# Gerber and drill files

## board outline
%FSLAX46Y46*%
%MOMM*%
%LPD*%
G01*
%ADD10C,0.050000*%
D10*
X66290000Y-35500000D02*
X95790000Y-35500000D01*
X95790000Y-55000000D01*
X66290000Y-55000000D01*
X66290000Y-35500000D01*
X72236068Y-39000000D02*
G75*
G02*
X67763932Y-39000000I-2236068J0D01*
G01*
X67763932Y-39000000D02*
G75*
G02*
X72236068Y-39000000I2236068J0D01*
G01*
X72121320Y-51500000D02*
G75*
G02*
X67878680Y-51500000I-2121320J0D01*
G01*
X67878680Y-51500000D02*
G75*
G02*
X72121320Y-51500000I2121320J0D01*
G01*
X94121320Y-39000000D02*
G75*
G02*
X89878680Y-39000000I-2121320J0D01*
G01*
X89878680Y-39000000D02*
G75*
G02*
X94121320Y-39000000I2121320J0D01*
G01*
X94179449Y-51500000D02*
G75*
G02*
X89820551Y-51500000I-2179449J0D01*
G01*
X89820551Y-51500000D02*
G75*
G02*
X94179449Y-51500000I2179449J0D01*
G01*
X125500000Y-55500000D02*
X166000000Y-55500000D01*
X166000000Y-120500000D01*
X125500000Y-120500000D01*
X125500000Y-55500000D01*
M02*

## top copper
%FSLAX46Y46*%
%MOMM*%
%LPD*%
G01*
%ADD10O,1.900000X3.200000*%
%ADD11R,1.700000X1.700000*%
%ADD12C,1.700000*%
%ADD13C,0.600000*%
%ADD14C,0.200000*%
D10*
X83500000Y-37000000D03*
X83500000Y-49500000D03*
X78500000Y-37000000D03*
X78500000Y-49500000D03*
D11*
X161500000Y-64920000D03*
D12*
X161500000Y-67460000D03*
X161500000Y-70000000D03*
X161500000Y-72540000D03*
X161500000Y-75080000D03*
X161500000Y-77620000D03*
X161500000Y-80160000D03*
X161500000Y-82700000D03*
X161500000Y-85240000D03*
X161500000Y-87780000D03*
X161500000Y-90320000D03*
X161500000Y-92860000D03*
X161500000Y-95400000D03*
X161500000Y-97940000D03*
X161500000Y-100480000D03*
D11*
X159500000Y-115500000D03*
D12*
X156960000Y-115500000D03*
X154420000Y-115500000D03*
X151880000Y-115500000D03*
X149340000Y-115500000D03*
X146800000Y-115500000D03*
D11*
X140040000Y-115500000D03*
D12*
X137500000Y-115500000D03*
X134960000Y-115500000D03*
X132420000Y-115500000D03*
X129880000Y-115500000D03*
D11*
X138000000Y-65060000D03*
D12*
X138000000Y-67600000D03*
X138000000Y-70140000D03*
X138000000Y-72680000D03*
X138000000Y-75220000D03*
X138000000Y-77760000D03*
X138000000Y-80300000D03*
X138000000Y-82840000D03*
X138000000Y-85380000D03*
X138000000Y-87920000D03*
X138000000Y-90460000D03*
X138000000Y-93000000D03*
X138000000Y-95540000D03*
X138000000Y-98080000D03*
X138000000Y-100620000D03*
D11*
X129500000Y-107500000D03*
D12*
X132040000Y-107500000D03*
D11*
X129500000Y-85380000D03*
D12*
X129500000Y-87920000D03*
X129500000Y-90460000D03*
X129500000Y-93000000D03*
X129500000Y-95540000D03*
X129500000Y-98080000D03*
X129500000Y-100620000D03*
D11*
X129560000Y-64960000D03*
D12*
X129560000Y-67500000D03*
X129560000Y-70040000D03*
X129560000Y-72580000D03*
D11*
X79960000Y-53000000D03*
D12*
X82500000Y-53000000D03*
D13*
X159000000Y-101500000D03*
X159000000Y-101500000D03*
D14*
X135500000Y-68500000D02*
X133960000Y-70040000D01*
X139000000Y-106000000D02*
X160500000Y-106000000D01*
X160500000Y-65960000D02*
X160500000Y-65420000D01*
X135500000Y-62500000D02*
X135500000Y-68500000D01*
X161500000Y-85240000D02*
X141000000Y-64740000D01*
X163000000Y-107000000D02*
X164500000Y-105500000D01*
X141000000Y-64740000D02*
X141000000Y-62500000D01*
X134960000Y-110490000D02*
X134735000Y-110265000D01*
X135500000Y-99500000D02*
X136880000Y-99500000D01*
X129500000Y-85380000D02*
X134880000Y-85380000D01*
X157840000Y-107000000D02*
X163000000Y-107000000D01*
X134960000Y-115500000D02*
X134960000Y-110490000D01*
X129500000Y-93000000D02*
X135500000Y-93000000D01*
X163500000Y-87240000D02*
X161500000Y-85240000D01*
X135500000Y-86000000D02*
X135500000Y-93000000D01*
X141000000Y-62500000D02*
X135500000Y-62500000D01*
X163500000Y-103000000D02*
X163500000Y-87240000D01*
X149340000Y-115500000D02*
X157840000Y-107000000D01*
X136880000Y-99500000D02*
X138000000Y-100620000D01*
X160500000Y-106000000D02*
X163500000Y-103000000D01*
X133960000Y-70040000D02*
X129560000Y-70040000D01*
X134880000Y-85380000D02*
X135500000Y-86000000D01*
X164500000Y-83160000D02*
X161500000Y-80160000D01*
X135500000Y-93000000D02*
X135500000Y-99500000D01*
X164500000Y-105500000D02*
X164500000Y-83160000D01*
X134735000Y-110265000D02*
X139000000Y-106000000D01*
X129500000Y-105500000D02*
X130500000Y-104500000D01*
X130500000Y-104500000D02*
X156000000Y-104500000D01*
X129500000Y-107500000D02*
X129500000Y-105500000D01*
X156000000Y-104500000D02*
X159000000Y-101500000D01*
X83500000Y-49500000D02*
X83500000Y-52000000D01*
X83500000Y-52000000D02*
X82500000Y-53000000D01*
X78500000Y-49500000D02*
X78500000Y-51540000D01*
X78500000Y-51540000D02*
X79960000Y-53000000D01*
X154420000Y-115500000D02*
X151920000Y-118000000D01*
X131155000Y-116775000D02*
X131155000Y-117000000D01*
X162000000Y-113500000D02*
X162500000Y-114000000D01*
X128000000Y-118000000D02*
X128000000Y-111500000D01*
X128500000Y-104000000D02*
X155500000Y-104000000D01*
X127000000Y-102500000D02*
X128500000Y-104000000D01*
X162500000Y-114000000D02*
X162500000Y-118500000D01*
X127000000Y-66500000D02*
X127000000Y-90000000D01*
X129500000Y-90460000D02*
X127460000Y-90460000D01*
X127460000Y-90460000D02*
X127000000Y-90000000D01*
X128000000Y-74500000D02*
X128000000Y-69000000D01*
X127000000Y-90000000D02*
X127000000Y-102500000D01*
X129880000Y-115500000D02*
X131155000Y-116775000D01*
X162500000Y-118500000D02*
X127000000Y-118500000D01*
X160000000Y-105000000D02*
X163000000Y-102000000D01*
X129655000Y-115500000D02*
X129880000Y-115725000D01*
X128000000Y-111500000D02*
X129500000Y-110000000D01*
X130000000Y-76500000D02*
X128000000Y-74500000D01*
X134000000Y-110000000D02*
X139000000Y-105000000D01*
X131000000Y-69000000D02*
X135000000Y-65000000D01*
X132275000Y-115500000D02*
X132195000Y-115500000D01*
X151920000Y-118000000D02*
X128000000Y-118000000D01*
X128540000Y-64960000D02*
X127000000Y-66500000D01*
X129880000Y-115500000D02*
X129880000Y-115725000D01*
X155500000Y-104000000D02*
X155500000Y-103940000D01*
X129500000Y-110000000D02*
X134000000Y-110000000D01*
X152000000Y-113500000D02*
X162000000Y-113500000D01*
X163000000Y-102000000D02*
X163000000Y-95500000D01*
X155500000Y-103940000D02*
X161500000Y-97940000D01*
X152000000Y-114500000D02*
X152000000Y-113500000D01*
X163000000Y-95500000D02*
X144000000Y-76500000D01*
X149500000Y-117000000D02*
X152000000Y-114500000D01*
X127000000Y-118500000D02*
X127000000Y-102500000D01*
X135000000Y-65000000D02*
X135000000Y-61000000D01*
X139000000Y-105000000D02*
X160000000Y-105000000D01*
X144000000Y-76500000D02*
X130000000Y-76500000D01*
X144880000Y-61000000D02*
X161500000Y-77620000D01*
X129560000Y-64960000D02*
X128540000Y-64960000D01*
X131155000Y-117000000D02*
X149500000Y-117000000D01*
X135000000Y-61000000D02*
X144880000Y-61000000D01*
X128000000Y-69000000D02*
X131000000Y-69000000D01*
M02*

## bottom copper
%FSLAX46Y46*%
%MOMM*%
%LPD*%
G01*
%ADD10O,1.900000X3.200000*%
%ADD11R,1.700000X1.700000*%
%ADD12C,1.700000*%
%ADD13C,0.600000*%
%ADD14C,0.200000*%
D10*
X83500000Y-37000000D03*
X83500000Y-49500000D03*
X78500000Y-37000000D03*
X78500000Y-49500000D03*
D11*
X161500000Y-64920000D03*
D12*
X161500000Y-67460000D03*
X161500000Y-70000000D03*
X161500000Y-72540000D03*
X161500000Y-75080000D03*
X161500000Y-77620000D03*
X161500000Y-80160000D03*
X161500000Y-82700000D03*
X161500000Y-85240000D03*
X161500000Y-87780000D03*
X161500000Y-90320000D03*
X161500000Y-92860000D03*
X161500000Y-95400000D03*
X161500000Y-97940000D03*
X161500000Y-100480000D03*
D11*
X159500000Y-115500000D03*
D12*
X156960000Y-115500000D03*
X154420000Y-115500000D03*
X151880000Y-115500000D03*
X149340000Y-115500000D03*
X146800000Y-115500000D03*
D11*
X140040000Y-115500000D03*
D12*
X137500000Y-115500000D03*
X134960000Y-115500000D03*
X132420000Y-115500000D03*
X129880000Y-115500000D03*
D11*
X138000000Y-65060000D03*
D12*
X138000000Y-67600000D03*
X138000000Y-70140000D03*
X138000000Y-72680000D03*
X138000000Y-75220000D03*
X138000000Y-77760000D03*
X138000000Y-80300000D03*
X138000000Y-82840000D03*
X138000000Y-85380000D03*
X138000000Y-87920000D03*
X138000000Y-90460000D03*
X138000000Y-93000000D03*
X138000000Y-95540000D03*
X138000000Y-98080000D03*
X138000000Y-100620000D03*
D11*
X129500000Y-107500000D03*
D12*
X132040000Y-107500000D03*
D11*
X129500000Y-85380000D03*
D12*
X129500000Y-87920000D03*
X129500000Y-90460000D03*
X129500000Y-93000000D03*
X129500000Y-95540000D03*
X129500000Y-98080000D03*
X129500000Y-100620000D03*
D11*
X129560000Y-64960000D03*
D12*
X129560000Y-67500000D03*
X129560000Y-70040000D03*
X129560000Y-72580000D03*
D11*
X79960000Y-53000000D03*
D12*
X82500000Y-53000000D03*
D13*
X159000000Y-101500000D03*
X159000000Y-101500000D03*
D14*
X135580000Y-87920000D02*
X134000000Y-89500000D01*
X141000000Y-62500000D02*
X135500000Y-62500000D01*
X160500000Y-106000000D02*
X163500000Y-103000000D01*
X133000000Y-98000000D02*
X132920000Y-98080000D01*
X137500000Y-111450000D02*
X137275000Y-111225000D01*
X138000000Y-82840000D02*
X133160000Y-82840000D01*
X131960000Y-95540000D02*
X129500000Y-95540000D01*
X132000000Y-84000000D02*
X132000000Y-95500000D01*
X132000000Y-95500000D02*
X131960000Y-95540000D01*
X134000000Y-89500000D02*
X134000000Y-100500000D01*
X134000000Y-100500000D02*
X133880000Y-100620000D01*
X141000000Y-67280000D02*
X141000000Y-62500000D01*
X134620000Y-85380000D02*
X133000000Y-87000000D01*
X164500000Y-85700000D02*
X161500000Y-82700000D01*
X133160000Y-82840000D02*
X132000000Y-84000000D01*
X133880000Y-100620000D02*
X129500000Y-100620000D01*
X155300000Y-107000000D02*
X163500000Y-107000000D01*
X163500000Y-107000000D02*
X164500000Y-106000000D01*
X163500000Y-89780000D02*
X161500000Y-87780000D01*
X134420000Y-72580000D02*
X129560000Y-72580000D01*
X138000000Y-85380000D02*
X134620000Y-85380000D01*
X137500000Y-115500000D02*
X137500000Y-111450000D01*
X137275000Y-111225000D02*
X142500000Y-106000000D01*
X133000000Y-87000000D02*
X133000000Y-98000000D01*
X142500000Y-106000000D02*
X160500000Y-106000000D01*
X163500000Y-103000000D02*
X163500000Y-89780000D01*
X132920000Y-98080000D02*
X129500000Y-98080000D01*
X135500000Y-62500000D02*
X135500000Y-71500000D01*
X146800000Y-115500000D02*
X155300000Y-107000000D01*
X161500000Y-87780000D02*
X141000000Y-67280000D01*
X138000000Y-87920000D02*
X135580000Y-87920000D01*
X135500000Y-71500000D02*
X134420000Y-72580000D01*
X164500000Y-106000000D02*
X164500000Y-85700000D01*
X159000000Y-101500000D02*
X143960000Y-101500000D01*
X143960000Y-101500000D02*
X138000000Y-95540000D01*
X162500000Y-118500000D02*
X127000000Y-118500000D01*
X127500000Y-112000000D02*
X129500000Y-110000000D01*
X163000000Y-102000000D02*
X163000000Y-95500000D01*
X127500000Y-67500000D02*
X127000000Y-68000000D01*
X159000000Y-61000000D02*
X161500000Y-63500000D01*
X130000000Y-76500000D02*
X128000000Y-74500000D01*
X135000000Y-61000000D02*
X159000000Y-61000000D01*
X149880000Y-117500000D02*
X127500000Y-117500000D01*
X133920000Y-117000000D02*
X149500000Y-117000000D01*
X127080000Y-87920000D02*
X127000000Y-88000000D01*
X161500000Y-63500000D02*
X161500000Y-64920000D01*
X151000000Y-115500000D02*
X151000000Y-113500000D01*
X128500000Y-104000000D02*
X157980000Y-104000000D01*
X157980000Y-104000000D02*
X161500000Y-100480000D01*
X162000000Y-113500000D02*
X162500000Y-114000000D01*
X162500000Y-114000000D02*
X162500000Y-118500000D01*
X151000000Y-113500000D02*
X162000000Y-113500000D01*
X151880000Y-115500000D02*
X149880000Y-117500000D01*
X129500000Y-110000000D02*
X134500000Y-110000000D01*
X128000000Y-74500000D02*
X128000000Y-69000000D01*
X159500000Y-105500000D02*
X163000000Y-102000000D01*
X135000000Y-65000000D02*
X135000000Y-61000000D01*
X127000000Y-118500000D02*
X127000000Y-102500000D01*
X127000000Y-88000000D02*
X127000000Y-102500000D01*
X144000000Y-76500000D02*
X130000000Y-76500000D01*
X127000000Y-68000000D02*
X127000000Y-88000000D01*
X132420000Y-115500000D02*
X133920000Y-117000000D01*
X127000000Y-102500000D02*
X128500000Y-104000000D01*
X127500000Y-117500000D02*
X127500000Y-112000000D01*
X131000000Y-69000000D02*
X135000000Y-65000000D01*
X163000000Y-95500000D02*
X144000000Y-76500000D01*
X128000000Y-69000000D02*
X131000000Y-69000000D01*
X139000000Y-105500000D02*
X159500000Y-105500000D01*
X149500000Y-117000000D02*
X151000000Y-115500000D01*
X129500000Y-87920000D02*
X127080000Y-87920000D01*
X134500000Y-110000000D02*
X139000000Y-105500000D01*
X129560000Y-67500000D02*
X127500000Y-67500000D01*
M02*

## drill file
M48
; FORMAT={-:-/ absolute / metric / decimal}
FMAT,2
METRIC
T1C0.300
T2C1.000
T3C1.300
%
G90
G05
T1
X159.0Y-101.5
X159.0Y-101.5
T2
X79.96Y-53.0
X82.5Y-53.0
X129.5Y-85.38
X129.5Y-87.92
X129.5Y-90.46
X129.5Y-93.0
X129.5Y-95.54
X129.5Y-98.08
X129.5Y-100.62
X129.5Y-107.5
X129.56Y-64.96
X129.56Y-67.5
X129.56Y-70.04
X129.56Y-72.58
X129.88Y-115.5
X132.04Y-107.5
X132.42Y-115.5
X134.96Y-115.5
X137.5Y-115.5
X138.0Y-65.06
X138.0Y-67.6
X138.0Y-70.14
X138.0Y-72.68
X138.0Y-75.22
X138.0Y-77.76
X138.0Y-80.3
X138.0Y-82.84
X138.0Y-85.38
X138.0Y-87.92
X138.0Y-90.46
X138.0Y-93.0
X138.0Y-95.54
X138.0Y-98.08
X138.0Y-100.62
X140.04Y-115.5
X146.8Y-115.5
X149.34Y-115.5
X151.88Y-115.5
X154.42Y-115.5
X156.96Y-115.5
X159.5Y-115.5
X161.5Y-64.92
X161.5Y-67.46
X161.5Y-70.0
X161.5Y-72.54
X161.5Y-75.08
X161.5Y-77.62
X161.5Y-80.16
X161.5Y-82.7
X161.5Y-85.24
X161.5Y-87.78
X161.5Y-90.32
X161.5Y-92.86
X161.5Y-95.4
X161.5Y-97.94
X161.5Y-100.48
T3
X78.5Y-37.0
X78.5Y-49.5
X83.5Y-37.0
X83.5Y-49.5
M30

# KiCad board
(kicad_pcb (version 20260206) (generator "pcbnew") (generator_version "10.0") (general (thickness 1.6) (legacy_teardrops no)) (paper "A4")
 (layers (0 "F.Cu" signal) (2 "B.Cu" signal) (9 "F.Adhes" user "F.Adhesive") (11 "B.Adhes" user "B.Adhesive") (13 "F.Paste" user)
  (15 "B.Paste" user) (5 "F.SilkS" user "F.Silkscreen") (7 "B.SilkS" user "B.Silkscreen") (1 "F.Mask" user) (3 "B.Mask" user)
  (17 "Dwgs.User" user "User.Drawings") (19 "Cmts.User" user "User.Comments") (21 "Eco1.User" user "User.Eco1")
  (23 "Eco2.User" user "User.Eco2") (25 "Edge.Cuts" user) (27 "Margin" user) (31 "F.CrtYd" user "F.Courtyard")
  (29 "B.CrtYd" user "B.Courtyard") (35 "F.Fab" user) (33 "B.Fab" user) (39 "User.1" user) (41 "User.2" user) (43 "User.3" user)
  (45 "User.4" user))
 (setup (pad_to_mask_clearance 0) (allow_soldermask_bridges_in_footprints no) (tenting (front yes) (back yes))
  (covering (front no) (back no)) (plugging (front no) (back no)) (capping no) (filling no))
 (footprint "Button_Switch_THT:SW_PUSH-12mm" (layer "F.Cu") (at 83.5 37 -90)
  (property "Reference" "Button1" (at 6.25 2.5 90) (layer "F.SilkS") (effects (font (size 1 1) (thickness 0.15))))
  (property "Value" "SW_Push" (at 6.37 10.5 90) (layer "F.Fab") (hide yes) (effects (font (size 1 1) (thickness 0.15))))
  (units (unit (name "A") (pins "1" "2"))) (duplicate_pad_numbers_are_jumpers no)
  (pad "1" thru_hole oval (at 0 0 270) (size 3.2 1.9) (drill 1.3) (layers "*.Cu" "*.Mask") (remove_unused_layers no)
   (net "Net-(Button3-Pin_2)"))
  (pad "1" thru_hole oval (at 12.5 0 270) (size 3.2 1.9) (drill 1.3) (layers "*.Cu" "*.Mask") (remove_unused_layers no)
   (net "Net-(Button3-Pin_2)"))
  (pad "2" thru_hole oval (at 0 5 270) (size 3.2 1.9) (drill 1.3) (layers "*.Cu" "*.Mask") (remove_unused_layers no)
   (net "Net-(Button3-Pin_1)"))
  (pad "2" thru_hole oval (at 12.5 5 270) (size 3.2 1.9) (drill 1.3) (layers "*.Cu" "*.Mask") (remove_unused_layers no)
   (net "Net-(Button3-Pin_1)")))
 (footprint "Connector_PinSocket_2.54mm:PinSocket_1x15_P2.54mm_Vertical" (layer "F.Cu") (at 161.5 64.92)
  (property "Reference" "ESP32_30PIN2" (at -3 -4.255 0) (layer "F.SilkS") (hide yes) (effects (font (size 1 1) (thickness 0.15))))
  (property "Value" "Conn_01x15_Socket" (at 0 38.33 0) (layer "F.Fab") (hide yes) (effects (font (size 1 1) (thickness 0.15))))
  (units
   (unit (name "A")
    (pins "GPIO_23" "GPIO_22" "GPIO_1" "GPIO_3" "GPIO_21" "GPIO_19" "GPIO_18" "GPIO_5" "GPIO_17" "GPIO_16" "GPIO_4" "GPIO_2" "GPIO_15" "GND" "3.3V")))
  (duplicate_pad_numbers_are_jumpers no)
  (pad "1" thru_hole rect (at 0 0) (size 1.7 1.7) (drill 1) (layers "*.Cu" "*.Mask") (remove_unused_layers no))
  (pad "2" thru_hole circle (at 0 2.54) (size 1.7 1.7) (drill 1) (layers "*.Cu" "*.Mask") (remove_unused_layers no))
  (pad "3" thru_hole circle (at 0 5.08) (size 1.7 1.7) (drill 1) (layers "*.Cu" "*.Mask") (remove_unused_layers no))
  (pad "4" thru_hole circle (at 0 7.62) (size 1.7 1.7) (drill 1) (layers "*.Cu" "*.Mask") (remove_unused_layers no))
  (pad "5" thru_hole circle (at 0 10.16) (size 1.7 1.7) (drill 1) (layers "*.Cu" "*.Mask") (remove_unused_layers no))
  (pad "6" thru_hole circle (at 0 12.7) (size 1.7 1.7) (drill 1) (layers "*.Cu" "*.Mask") (remove_unused_layers no))
  (pad "7" thru_hole circle (at 0 15.24) (size 1.7 1.7) (drill 1) (layers "*.Cu" "*.Mask") (remove_unused_layers no))
  (pad "8" thru_hole circle (at 0 17.78) (size 1.7 1.7) (drill 1) (layers "*.Cu" "*.Mask") (remove_unused_layers no))
  (pad "9" thru_hole circle (at 0 20.32) (size 1.7 1.7) (drill 1) (layers "*.Cu" "*.Mask") (remove_unused_layers no))
  (pad "10" thru_hole circle (at 0 22.86) (size 1.7 1.7) (drill 1) (layers "*.Cu" "*.Mask") (remove_unused_layers no))
  (pad "11" thru_hole circle (at 0 25.4) (size 1.7 1.7) (drill 1) (layers "*.Cu" "*.Mask") (remove_unused_layers no))
  (pad "12" thru_hole circle (at 0 27.94) (size 1.7 1.7) (drill 1) (layers "*.Cu" "*.Mask") (remove_unused_layers no))
  (pad "13" thru_hole circle (at 0 30.48) (size 1.7 1.7) (drill 1) (layers "*.Cu" "*.Mask") (remove_unused_layers no))
  (pad "14" thru_hole circle (at 0 33.02) (size 1.7 1.7) (drill 1) (layers "*.Cu" "*.Mask") (remove_unused_layers no))
  (pad "15" thru_hole circle (at 0 35.56) (size 1.7 1.7) (drill 1) (layers "*.Cu" "*.Mask") (remove_unused_layers no)))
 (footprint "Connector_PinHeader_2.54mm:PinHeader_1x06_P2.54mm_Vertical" (layer "F.Cu") (at 159.5 115.5 -90)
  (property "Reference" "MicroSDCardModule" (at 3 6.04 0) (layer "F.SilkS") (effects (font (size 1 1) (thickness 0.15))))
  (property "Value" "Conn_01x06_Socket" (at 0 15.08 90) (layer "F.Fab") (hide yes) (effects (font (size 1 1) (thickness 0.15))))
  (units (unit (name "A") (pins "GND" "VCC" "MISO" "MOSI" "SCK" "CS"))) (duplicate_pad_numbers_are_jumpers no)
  (pad "1" thru_hole rect (at 0 0 270) (size 1.7 1.7) (drill 1) (layers "*.Cu" "*.Mask") (remove_unused_layers no))
  (pad "2" thru_hole circle (at 0 2.54 270) (size 1.7 1.7) (drill 1) (layers "*.Cu" "*.Mask") (remove_unused_layers no))
  (pad "3" thru_hole circle (at 0 5.08 270) (size 1.7 1.7) (drill 1) (layers "*.Cu" "*.Mask") (remove_unused_layers no))
  (pad "4" thru_hole circle (at 0 7.62 270) (size 1.7 1.7) (drill 1) (layers "*.Cu" "*.Mask") (remove_unused_layers no))
  (pad "5" thru_hole circle (at 0 10.16 270) (size 1.7 1.7) (drill 1) (layers "*.Cu" "*.Mask") (remove_unused_layers no))
  (pad "6" thru_hole circle (at 0 12.7 270) (size 1.7 1.7) (drill 1) (layers "*.Cu" "*.Mask") (remove_unused_layers no)))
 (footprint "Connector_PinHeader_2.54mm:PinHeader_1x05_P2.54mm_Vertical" (layer "F.Cu") (at 140.04 115.5 -90)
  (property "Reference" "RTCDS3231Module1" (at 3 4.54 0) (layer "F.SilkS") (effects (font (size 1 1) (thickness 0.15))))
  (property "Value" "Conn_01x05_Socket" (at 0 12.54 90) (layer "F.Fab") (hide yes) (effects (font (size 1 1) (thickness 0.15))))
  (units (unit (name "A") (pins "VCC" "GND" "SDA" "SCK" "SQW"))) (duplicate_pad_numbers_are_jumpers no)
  (pad "1" thru_hole rect (at 0 0 270) (size 1.7 1.7) (drill 1) (layers "*.Cu" "*.Mask") (remove_unused_layers no))
  (pad "2" thru_hole circle (at 0 2.54 270) (size 1.7 1.7) (drill 1) (layers "*.Cu" "*.Mask") (remove_unused_layers no))
  (pad "3" thru_hole circle (at 0 5.08 270) (size 1.7 1.7) (drill 1) (layers "*.Cu" "*.Mask") (remove_unused_layers no))
  (pad "4" thru_hole circle (at 0 7.62 270) (size 1.7 1.7) (drill 1) (layers "*.Cu" "*.Mask") (remove_unused_layers no))
  (pad "5" thru_hole circle (at 0 10.16 270) (size 1.7 1.7) (drill 1) (layers "*.Cu" "*.Mask") (remove_unused_layers no)))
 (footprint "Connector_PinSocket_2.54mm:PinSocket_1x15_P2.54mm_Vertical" (layer "F.Cu") (at 138 65.06)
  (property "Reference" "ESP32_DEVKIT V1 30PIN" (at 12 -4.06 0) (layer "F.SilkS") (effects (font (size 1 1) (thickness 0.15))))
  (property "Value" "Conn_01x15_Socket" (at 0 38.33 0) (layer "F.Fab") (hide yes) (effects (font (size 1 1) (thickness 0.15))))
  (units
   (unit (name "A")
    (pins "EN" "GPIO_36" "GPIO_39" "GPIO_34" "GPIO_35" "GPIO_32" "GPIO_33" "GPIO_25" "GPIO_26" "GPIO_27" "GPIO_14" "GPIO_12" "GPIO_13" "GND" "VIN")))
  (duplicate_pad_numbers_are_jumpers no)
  (pad "1" thru_hole rect (at 0 0) (size 1.7 1.7) (drill 1) (layers "*.Cu" "*.Mask") (remove_unused_layers no))
  (pad "2" thru_hole circle (at 0 2.54) (size 1.7 1.7) (drill 1) (layers "*.Cu" "*.Mask") (remove_unused_layers no))
  (pad "3" thru_hole circle (at 0 5.08) (size 1.7 1.7) (drill 1) (layers "*.Cu" "*.Mask") (remove_unused_layers no))
  (pad "4" thru_hole circle (at 0 7.62) (size 1.7 1.7) (drill 1) (layers "*.Cu" "*.Mask") (remove_unused_layers no))
  (pad "5" thru_hole circle (at 0 10.16) (size 1.7 1.7) (drill 1) (layers "*.Cu" "*.Mask") (remove_unused_layers no))
  (pad "6" thru_hole circle (at 0 12.7) (size 1.7 1.7) (drill 1) (layers "*.Cu" "*.Mask") (remove_unused_layers no))
  (pad "7" thru_hole circle (at 0 15.24) (size 1.7 1.7) (drill 1) (layers "*.Cu" "*.Mask") (remove_unused_layers no))
  (pad "8" thru_hole circle (at 0 17.78) (size 1.7 1.7) (drill 1) (layers "*.Cu" "*.Mask") (remove_unused_layers no))
  (pad "9" thru_hole circle (at 0 20.32) (size 1.7 1.7) (drill 1) (layers "*.Cu" "*.Mask") (remove_unused_layers no))
  (pad "10" thru_hole circle (at 0 22.86) (size 1.7 1.7) (drill 1) (layers "*.Cu" "*.Mask") (remove_unused_layers no))
  (pad "11" thru_hole circle (at 0 25.4) (size 1.7 1.7) (drill 1) (layers "*.Cu" "*.Mask") (remove_unused_layers no))
  (pad "12" thru_hole circle (at 0 27.94) (size 1.7 1.7) (drill 1) (layers "*.Cu" "*.Mask") (remove_unused_layers no))
  (pad "13" thru_hole circle (at 0 30.48) (size 1.7 1.7) (drill 1) (layers "*.Cu" "*.Mask") (remove_unused_layers no))
  (pad "14" thru_hole circle (at 0 33.02) (size 1.7 1.7) (drill 1) (layers "*.Cu" "*.Mask") (remove_unused_layers no))
  (pad "15" thru_hole circle (at 0 35.56) (size 1.7 1.7) (drill 1) (layers "*.Cu" "*.Mask") (remove_unused_layers no)))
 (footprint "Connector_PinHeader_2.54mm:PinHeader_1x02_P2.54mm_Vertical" (layer "F.Cu") (at 129.5 107.5 90)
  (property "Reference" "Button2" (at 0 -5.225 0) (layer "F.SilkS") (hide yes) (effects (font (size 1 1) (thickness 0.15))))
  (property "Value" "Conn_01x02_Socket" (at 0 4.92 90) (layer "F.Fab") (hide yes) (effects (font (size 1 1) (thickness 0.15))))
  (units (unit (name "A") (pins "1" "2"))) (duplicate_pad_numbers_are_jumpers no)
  (pad "1" thru_hole rect (at 0 0 90) (size 1.7 1.7) (drill 1) (layers "*.Cu" "*.Mask") (remove_unused_layers no))
  (pad "2" thru_hole circle (at 0 2.54 90) (size 1.7 1.7) (drill 1) (layers "*.Cu" "*.Mask") (remove_unused_layers no)))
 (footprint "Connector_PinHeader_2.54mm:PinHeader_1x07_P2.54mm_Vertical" (layer "F.Cu") (at 129.5 85.38)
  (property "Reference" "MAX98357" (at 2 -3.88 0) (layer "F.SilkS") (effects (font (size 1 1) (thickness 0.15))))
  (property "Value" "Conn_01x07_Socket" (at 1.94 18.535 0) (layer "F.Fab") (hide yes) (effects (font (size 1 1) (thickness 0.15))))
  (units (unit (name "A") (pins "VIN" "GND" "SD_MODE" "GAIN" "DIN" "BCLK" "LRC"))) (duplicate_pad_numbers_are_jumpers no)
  (pad "1" thru_hole rect (at 0 0) (size 1.7 1.7) (drill 1) (layers "*.Cu" "*.Mask") (remove_unused_layers no))
  (pad "2" thru_hole circle (at 0 2.54) (size 1.7 1.7) (drill 1) (layers "*.Cu" "*.Mask") (remove_unused_layers no))
  (pad "3" thru_hole circle (at 0 5.08) (size 1.7 1.7) (drill 1) (layers "*.Cu" "*.Mask") (remove_unused_layers no))
  (pad "4" thru_hole circle (at 0 7.62) (size 1.7 1.7) (drill 1) (layers "*.Cu" "*.Mask") (remove_unused_layers no))
  (pad "5" thru_hole circle (at 0 10.16) (size 1.7 1.7) (drill 1) (layers "*.Cu" "*.Mask") (remove_unused_layers no))
  (pad "6" thru_hole circle (at 0 12.7) (size 1.7 1.7) (drill 1) (layers "*.Cu" "*.Mask") (remove_unused_layers no))
  (pad "7" thru_hole circle (at 0 15.24) (size 1.7 1.7) (drill 1) (layers "*.Cu" "*.Mask") (remove_unused_layers no)))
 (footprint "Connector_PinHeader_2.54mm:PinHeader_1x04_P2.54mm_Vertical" (layer "F.Cu") (at 129.56 64.96)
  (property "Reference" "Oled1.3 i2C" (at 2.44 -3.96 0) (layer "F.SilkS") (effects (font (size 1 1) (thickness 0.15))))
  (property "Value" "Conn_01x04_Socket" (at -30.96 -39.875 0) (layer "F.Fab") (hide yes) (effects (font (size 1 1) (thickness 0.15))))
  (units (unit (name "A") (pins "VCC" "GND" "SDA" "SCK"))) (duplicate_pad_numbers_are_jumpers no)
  (pad "1" thru_hole rect (at 0 0) (size 1.7 1.7) (drill 1) (layers "*.Cu" "*.Mask") (remove_unused_layers no))
  (pad "2" thru_hole circle (at 0 2.54) (size 1.7 1.7) (drill 1) (layers "*.Cu" "*.Mask") (remove_unused_layers no))
  (pad "3" thru_hole circle (at 0 5.08) (size 1.7 1.7) (drill 1) (layers "*.Cu" "*.Mask") (remove_unused_layers no))
  (pad "4" thru_hole circle (at 0 7.62) (size 1.7 1.7) (drill 1) (layers "*.Cu" "*.Mask") (remove_unused_layers no)))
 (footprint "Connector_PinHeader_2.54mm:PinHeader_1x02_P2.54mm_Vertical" (layer "B.Cu") (at 79.96 53 -90)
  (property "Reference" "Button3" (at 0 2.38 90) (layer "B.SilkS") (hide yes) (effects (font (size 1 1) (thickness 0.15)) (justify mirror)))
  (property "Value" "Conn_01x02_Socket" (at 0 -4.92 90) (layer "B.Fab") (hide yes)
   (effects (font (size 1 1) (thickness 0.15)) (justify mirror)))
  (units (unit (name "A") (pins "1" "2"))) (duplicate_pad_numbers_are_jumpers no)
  (pad "1" thru_hole rect (at 0 0 270) (size 1.7 1.7) (drill 1) (layers "*.Cu" "*.Mask") (remove_unused_layers no)
   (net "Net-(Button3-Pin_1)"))
  (pad "2" thru_hole circle (at 0 -2.54 270) (size 1.7 1.7) (drill 1) (layers "*.Cu" "*.Mask") (remove_unused_layers no)
   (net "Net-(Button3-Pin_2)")))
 (gr_rect (start 66.29 35.5) (end 95.79 55) (stroke (width 0.05) (type default)) (fill no) (layer "Edge.Cuts"))
 (gr_circle (center 70 39) (end 72 38) (stroke (width 0.05) (type default)) (fill no) (layer "Edge.Cuts"))
 (gr_circle (center 70 51.5) (end 71.5 50) (stroke (width 0.05) (type default)) (fill no) (layer "Edge.Cuts"))
 (gr_circle (center 92 39) (end 93.5 37.5) (stroke (width 0.05) (type default)) (fill no) (layer "Edge.Cuts"))
 (gr_circle (center 92 51.5) (end 94.12132 51) (stroke (width 0.05) (type default)) (fill no) (layer "Edge.Cuts"))
 (gr_rect (start 125.5 55.5) (end 166 120.5) (stroke (width 0.05) (type default)) (fill no) (layer "Edge.Cuts"))
 (segment (start 135.5 68.5) (end 133.96 70.04) (width 0.2) (layer "F.Cu") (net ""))
 (segment (start 139 106) (end 160.5 106) (width 0.2) (layer "F.Cu") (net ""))
 (segment (start 160.5 65.96) (end 160.5 65.42) (width 0.2) (layer "F.Cu") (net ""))
 (segment (start 135.5 62.5) (end 135.5 68.5) (width 0.2) (layer "F.Cu") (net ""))
 (segment (start 161.5 85.24) (end 141 64.74) (width 0.2) (layer "F.Cu") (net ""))
 (segment (start 163 107) (end 164.5 105.5) (width 0.2) (layer "F.Cu") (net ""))
 (segment (start 141 64.74) (end 141 62.5) (width 0.2) (layer "F.Cu") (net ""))
 (segment (start 134.96 110.49) (end 134.735 110.265) (width 0.2) (layer "F.Cu") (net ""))
 (segment (start 135.5 99.5) (end 136.88 99.5) (width 0.2) (layer "F.Cu") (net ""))
 (segment (start 129.5 85.38) (end 134.88 85.38) (width 0.2) (layer "F.Cu") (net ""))
 (segment (start 157.84 107) (end 163 107) (width 0.2) (layer "F.Cu") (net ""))
 (segment (start 134.96 115.5) (end 134.96 110.49) (width 0.2) (layer "F.Cu") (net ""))
 (segment (start 129.5 93) (end 135.5 93) (width 0.2) (layer "F.Cu") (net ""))
 (segment (start 163.5 87.24) (end 161.5 85.24) (width 0.2) (layer "F.Cu") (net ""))
 (segment (start 135.5 86) (end 135.5 93) (width 0.2) (layer "F.Cu") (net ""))
 (segment (start 141 62.5) (end 135.5 62.5) (width 0.2) (layer "F.Cu") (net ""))
 (segment (start 163.5 103) (end 163.5 87.24) (width 0.2) (layer "F.Cu") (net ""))
 (segment (start 149.34 115.5) (end 157.84 107) (width 0.2) (layer "F.Cu") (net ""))
 (segment (start 136.88 99.5) (end 138 100.62) (width 0.2) (layer "F.Cu") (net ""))
 (segment (start 160.5 106) (end 163.5 103) (width 0.2) (layer "F.Cu") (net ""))
 (segment (start 133.96 70.04) (end 129.56 70.04) (width 0.2) (layer "F.Cu") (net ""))
 (segment (start 134.88 85.38) (end 135.5 86) (width 0.2) (layer "F.Cu") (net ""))
 (segment (start 164.5 83.16) (end 161.5 80.16) (width 0.2) (layer "F.Cu") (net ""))
 (segment (start 135.5 93) (end 135.5 99.5) (width 0.2) (layer "F.Cu") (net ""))
 (segment (start 164.5 105.5) (end 164.5 83.16) (width 0.2) (layer "F.Cu") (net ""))
 (segment (start 134.735 110.265) (end 139 106) (width 0.2) (layer "F.Cu") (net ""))
 (segment (start 135.58 87.92) (end 134 89.5) (width 0.2) (layer "B.Cu") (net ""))
 (segment (start 141 62.5) (end 135.5 62.5) (width 0.2) (layer "B.Cu") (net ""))
 (segment (start 160.5 106) (end 163.5 103) (width 0.2) (layer "B.Cu") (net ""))
 (segment (start 133 98) (end 132.92 98.08) (width 0.2) (layer "B.Cu") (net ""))
 (segment (start 137.5 111.45) (end 137.275 111.225) (width 0.2) (layer "B.Cu") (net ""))
 (segment (start 138 82.84) (end 133.16 82.84) (width 0.2) (layer "B.Cu") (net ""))
 (segment (start 131.96 95.54) (end 129.5 95.54) (width 0.2) (layer "B.Cu") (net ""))
 (segment (start 132 84) (end 132 95.5) (width 0.2) (layer "B.Cu") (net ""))
 (segment (start 132 95.5) (end 131.96 95.54) (width 0.2) (layer "B.Cu") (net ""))
 (segment (start 134 89.5) (end 134 100.5) (width 0.2) (layer "B.Cu") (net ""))
 (segment (start 134 100.5) (end 133.88 100.62) (width 0.2) (layer "B.Cu") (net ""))
 (segment (start 141 67.28) (end 141 62.5) (width 0.2) (layer "B.Cu") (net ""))
 (segment (start 134.62 85.38) (end 133 87) (width 0.2) (layer "B.Cu") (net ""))
 (segment (start 164.5 85.7) (end 161.5 82.7) (width 0.2) (layer "B.Cu") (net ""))
 (segment (start 133.16 82.84) (end 132 84) (width 0.2) (layer "B.Cu") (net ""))
 (segment (start 133.88 100.62) (end 129.5 100.62) (width 0.2) (layer "B.Cu") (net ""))
 (segment (start 155.3 107) (end 163.5 107) (width 0.2) (layer "B.Cu") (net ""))
 (segment (start 163.5 107) (end 164.5 106) (width 0.2) (layer "B.Cu") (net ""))
 (segment (start 163.5 89.78) (end 161.5 87.78) (width 0.2) (layer "B.Cu") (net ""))
 (segment (start 134.42 72.58) (end 129.56 72.58) (width 0.2) (layer "B.Cu") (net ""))
 (segment (start 138 85.38) (end 134.62 85.38) (width 0.2) (layer "B.Cu") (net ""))
 (segment (start 137.5 115.5) (end 137.5 111.45) (width 0.2) (layer "B.Cu") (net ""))
 (segment (start 137.275 111.225) (end 142.5 106) (width 0.2) (layer "B.Cu") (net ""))
 (segment (start 133 87) (end 133 98) (width 0.2) (layer "B.Cu") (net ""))
 (segment (start 142.5 106) (end 160.5 106) (width 0.2) (layer "B.Cu") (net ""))
 (segment (start 163.5 103) (end 163.5 89.78) (width 0.2) (layer "B.Cu") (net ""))
 (segment (start 132.92 98.08) (end 129.5 98.08) (width 0.2) (layer "B.Cu") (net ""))
 (segment (start 135.5 62.5) (end 135.5 71.5) (width 0.2) (layer "B.Cu") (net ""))
 (segment (start 146.8 115.5) (end 155.3 107) (width 0.2) (layer "B.Cu") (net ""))
 (segment (start 161.5 87.78) (end 141 67.28) (width 0.2) (layer "B.Cu") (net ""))
 (segment (start 138 87.92) (end 135.58 87.92) (width 0.2) (layer "B.Cu") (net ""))
 (segment (start 135.5 71.5) (end 134.42 72.58) (width 0.2) (layer "B.Cu") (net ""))
 (segment (start 164.5 106) (end 164.5 85.7) (width 0.2) (layer "B.Cu") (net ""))
 (segment (start 129.5 105.5) (end 130.5 104.5) (width 0.2) (layer "F.Cu") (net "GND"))
 (segment (start 130.5 104.5) (end 156 104.5) (width 0.2) (layer "F.Cu") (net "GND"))
 (segment (start 129.5 107.5) (end 129.5 105.5) (width 0.2) (layer "F.Cu") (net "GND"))
 (segment (start 156 104.5) (end 159 101.5) (width 0.2) (layer "F.Cu") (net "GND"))
 (via (at 159 101.5) (size 0.6) (drill 0.3) (layers "F.Cu" "B.Cu") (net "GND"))
 (via (at 159 101.5) (size 0.6) (drill 0.3) (layers "F.Cu" "B.Cu") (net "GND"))
 (segment (start 159 101.5) (end 143.96 101.5) (width 0.2) (layer "B.Cu") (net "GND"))
 (segment (start 143.96 101.5) (end 138 95.54) (width 0.2) (layer "B.Cu") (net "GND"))
 (segment (start 83.5 49.5) (end 83.5 52) (width 0.2) (layer "F.Cu") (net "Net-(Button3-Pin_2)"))
 (segment (start 83.5 52) (end 82.5 53) (width 0.2) (layer "F.Cu") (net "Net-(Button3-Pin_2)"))
 (segment (start 78.5 49.5) (end 78.5 51.54) (width 0.2) (layer "F.Cu") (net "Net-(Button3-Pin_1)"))
 (segment (start 78.5 51.54) (end 79.96 53) (width 0.2) (layer "F.Cu") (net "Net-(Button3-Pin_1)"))
 (segment (start 154.42 115.5) (end 151.92 118) (width 0.2) (layer "F.Cu") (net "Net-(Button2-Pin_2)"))
 (segment (start 131.155 116.775) (end 131.155 117) (width 0.2) (layer "F.Cu") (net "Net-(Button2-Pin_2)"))
 (segment (start 162 113.5) (end 162.5 114) (width 0.2) (layer "F.Cu") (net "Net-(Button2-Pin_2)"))
 (segment (start 128 118) (end 128 111.5) (width 0.2) (layer "F.Cu") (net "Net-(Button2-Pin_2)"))
 (segment (start 128.5 104) (end 155.5 104) (width 0.2) (layer "F.Cu") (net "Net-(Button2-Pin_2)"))
 (segment (start 127 102.5) (end 128.5 104) (width 0.2) (layer "F.Cu") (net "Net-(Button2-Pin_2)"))
 (segment (start 162.5 114) (end 162.5 118.5) (width 0.2) (layer "F.Cu") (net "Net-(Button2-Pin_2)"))
 (segment (start 127 66.5) (end 127 90) (width 0.2) (layer "F.Cu") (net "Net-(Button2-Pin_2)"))
 (segment (start 129.5 90.46) (end 127.46 90.46) (width 0.2) (layer "F.Cu") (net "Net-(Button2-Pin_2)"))
 (segment (start 127.46 90.46) (end 127 90) (width 0.2) (layer "F.Cu") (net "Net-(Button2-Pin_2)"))
 (segment (start 128 74.5) (end 128 69) (width 0.2) (layer "F.Cu") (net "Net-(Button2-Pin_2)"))
 (segment (start 127 90) (end 127 102.5) (width 0.2) (layer "F.Cu") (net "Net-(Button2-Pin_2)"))
 (segment (start 129.88 115.5) (end 131.155 116.775) (width 0.2) (layer "F.Cu") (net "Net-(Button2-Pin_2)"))
 (segment (start 162.5 118.5) (end 127 118.5) (width 0.2) (layer "F.Cu") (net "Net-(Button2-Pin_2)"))
 (segment (start 160 105) (end 163 102) (width 0.2) (layer "F.Cu") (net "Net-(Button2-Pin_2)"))
 (segment (start 129.655 115.5) (end 129.88 115.725) (width 0.2) (layer "F.Cu") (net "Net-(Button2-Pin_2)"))
 (segment (start 128 111.5) (end 129.5 110) (width 0.2) (layer "F.Cu") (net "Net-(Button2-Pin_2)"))
 (segment (start 130 76.5) (end 128 74.5) (width 0.2) (layer "F.Cu") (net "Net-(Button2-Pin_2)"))
 (segment (start 134 110) (end 139 105) (width 0.2) (layer "F.Cu") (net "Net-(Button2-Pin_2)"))
 (segment (start 131 69) (end 135 65) (width 0.2) (layer "F.Cu") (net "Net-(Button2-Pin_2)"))
 (segment (start 132.275 115.5) (end 132.195 115.5) (width 0.2) (layer "F.Cu") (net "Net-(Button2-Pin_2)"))
 (segment (start 151.92 118) (end 128 118) (width 0.2) (layer "F.Cu") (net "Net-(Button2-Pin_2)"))
 (segment (start 128.54 64.96) (end 127 66.5) (width 0.2) (layer "F.Cu") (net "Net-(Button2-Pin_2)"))
 (segment (start 129.88 115.5) (end 129.88 115.725) (width 0.2) (layer "F.Cu") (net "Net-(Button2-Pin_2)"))
 (segment (start 155.5 104) (end 155.5 103.94) (width 0.2) (layer "F.Cu") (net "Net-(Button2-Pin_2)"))
 (segment (start 129.5 110) (end 134 110) (width 0.2) (layer "F.Cu") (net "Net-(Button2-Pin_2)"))
 (segment (start 152 113.5) (end 162 113.5) (width 0.2) (layer "F.Cu") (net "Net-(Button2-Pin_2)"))
 (segment (start 163 102) (end 163 95.5) (width 0.2) (layer "F.Cu") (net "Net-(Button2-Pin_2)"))
 (segment (start 155.5 103.94) (end 161.5 97.94) (width 0.2) (layer "F.Cu") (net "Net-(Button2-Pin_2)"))
 (segment (start 152 114.5) (end 152 113.5) (width 0.2) (layer "F.Cu") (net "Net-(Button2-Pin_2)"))
 (segment (start 163 95.5) (end 144 76.5) (width 0.2) (layer "F.Cu") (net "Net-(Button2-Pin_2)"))
 (segment (start 149.5 117) (end 152 114.5) (width 0.2) (layer "F.Cu") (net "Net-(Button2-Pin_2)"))
 (segment (start 127 118.5) (end 127 102.5) (width 0.2) (layer "F.Cu") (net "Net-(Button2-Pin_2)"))
 (segment (start 135 65) (end 135 61) (width 0.2) (layer "F.Cu") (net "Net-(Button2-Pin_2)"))
 (segment (start 139 105) (end 160 105) (width 0.2) (layer "F.Cu") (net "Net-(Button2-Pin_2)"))
 (segment (start 144 76.5) (end 130 76.5) (width 0.2) (layer "F.Cu") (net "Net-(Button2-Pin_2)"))
 (segment (start 144.88 61) (end 161.5 77.62) (width 0.2) (layer "F.Cu") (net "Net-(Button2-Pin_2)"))
 (segment (start 129.56 64.96) (end 128.54 64.96) (width 0.2) (layer "F.Cu") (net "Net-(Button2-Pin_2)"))
 (segment (start 131.155 117) (end 149.5 117) (width 0.2) (layer "F.Cu") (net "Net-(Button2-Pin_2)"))
 (segment (start 135 61) (end 144.88 61) (width 0.2) (layer "F.Cu") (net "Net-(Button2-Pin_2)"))
 (segment (start 128 69) (end 131 69) (width 0.2) (layer "F.Cu") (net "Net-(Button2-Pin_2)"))
 (segment (start 162.5 118.5) (end 127 118.5) (width 0.2) (layer "B.Cu") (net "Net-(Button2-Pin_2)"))
 (segment (start 127.5 112) (end 129.5 110) (width 0.2) (layer "B.Cu") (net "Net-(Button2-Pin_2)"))
 (segment (start 163 102) (end 163 95.5) (width 0.2) (layer "B.Cu") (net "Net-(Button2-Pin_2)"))
 (segment (start 127.5 67.5) (end 127 68) (width 0.2) (layer "B.Cu") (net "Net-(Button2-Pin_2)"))
 (segment (start 159 61) (end 161.5 63.5) (width 0.2) (layer "B.Cu") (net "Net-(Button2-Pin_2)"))
 (segment (start 130 76.5) (end 128 74.5) (width 0.2) (layer "B.Cu") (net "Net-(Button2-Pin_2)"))
 (segment (start 135 61) (end 159 61) (width 0.2) (layer "B.Cu") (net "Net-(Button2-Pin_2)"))
 (segment (start 149.88 117.5) (end 127.5 117.5) (width 0.2) (layer "B.Cu") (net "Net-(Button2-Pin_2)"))
 (segment (start 133.92 117) (end 149.5 117) (width 0.2) (layer "B.Cu") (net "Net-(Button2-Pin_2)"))
 (segment (start 127.08 87.92) (end 127 88) (width 0.2) (layer "B.Cu") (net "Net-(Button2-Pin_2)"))
 (segment (start 161.5 63.5) (end 161.5 64.92) (width 0.2) (layer "B.Cu") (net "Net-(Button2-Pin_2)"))
 (segment (start 151 115.5) (end 151 113.5) (width 0.2) (layer "B.Cu") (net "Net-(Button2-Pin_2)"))
 (segment (start 128.5 104) (end 157.98 104) (width 0.2) (layer "B.Cu") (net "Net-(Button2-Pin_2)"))
 (segment (start 157.98 104) (end 161.5 100.48) (width 0.2) (layer "B.Cu") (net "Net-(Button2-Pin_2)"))
 (segment (start 162 113.5) (end 162.5 114) (width 0.2) (layer "B.Cu") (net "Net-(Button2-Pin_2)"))
 (segment (start 162.5 114) (end 162.5 118.5) (width 0.2) (layer "B.Cu") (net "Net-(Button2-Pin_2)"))
 (segment (start 151 113.5) (end 162 113.5) (width 0.2) (layer "B.Cu") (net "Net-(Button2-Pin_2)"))
 (segment (start 151.88 115.5) (end 149.88 117.5) (width 0.2) (layer "B.Cu") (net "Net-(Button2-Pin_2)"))
 (segment (start 129.5 110) (end 134.5 110) (width 0.2) (layer "B.Cu") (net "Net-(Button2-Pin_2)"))
 (segment (start 128 74.5) (end 128 69) (width 0.2) (layer "B.Cu") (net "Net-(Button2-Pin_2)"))
 (segment (start 159.5 105.5) (end 163 102) (width 0.2) (layer "B.Cu") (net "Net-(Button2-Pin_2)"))
 (segment (start 135 65) (end 135 61) (width 0.2) (layer "B.Cu") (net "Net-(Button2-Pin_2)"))
 (segment (start 127 118.5) (end 127 102.5) (width 0.2) (layer "B.Cu") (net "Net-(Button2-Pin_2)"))
 (segment (start 127 88) (end 127 102.5) (width 0.2) (layer "B.Cu") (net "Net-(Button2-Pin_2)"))
 (segment (start 144 76.5) (end 130 76.5) (width 0.2) (layer "B.Cu") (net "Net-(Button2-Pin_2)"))
 (segment (start 127 68) (end 127 88) (width 0.2) (layer "B.Cu") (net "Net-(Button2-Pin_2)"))
 (segment (start 132.42 115.5) (end 133.92 117) (width 0.2) (layer "B.Cu") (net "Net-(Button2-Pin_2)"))
 (segment (start 127 102.5) (end 128.5 104) (width 0.2) (layer "B.Cu") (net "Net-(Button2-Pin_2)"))
 (segment (start 127.5 117.5) (end 127.5 112) (width 0.2) (layer "B.Cu") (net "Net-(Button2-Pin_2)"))
 (segment (start 131 69) (end 135 65) (width 0.2) (layer "B.Cu") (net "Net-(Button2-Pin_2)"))
 (segment (start 163 95.5) (end 144 76.5) (width 0.2) (layer "B.Cu") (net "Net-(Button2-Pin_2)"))
 (segment (start 128 69) (end 131 69) (width 0.2) (layer "B.Cu") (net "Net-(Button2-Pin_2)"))
 (segment (start 139 105.5) (end 159.5 105.5) (width 0.2) (layer "B.Cu") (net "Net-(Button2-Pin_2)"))
 (segment (start 149.5 117) (end 151 115.5) (width 0.2) (layer "B.Cu") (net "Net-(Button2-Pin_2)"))
 (segment (start 129.5 87.92) (end 127.08 87.92) (width 0.2) (layer "B.Cu") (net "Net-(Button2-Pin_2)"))
 (segment (start 134.5 110) (end 139 105.5) (width 0.2) (layer "B.Cu") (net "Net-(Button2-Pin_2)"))
 (segment (start 129.56 67.5) (end 127.5 67.5) (width 0.2) (layer "B.Cu") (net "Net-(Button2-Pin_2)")))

